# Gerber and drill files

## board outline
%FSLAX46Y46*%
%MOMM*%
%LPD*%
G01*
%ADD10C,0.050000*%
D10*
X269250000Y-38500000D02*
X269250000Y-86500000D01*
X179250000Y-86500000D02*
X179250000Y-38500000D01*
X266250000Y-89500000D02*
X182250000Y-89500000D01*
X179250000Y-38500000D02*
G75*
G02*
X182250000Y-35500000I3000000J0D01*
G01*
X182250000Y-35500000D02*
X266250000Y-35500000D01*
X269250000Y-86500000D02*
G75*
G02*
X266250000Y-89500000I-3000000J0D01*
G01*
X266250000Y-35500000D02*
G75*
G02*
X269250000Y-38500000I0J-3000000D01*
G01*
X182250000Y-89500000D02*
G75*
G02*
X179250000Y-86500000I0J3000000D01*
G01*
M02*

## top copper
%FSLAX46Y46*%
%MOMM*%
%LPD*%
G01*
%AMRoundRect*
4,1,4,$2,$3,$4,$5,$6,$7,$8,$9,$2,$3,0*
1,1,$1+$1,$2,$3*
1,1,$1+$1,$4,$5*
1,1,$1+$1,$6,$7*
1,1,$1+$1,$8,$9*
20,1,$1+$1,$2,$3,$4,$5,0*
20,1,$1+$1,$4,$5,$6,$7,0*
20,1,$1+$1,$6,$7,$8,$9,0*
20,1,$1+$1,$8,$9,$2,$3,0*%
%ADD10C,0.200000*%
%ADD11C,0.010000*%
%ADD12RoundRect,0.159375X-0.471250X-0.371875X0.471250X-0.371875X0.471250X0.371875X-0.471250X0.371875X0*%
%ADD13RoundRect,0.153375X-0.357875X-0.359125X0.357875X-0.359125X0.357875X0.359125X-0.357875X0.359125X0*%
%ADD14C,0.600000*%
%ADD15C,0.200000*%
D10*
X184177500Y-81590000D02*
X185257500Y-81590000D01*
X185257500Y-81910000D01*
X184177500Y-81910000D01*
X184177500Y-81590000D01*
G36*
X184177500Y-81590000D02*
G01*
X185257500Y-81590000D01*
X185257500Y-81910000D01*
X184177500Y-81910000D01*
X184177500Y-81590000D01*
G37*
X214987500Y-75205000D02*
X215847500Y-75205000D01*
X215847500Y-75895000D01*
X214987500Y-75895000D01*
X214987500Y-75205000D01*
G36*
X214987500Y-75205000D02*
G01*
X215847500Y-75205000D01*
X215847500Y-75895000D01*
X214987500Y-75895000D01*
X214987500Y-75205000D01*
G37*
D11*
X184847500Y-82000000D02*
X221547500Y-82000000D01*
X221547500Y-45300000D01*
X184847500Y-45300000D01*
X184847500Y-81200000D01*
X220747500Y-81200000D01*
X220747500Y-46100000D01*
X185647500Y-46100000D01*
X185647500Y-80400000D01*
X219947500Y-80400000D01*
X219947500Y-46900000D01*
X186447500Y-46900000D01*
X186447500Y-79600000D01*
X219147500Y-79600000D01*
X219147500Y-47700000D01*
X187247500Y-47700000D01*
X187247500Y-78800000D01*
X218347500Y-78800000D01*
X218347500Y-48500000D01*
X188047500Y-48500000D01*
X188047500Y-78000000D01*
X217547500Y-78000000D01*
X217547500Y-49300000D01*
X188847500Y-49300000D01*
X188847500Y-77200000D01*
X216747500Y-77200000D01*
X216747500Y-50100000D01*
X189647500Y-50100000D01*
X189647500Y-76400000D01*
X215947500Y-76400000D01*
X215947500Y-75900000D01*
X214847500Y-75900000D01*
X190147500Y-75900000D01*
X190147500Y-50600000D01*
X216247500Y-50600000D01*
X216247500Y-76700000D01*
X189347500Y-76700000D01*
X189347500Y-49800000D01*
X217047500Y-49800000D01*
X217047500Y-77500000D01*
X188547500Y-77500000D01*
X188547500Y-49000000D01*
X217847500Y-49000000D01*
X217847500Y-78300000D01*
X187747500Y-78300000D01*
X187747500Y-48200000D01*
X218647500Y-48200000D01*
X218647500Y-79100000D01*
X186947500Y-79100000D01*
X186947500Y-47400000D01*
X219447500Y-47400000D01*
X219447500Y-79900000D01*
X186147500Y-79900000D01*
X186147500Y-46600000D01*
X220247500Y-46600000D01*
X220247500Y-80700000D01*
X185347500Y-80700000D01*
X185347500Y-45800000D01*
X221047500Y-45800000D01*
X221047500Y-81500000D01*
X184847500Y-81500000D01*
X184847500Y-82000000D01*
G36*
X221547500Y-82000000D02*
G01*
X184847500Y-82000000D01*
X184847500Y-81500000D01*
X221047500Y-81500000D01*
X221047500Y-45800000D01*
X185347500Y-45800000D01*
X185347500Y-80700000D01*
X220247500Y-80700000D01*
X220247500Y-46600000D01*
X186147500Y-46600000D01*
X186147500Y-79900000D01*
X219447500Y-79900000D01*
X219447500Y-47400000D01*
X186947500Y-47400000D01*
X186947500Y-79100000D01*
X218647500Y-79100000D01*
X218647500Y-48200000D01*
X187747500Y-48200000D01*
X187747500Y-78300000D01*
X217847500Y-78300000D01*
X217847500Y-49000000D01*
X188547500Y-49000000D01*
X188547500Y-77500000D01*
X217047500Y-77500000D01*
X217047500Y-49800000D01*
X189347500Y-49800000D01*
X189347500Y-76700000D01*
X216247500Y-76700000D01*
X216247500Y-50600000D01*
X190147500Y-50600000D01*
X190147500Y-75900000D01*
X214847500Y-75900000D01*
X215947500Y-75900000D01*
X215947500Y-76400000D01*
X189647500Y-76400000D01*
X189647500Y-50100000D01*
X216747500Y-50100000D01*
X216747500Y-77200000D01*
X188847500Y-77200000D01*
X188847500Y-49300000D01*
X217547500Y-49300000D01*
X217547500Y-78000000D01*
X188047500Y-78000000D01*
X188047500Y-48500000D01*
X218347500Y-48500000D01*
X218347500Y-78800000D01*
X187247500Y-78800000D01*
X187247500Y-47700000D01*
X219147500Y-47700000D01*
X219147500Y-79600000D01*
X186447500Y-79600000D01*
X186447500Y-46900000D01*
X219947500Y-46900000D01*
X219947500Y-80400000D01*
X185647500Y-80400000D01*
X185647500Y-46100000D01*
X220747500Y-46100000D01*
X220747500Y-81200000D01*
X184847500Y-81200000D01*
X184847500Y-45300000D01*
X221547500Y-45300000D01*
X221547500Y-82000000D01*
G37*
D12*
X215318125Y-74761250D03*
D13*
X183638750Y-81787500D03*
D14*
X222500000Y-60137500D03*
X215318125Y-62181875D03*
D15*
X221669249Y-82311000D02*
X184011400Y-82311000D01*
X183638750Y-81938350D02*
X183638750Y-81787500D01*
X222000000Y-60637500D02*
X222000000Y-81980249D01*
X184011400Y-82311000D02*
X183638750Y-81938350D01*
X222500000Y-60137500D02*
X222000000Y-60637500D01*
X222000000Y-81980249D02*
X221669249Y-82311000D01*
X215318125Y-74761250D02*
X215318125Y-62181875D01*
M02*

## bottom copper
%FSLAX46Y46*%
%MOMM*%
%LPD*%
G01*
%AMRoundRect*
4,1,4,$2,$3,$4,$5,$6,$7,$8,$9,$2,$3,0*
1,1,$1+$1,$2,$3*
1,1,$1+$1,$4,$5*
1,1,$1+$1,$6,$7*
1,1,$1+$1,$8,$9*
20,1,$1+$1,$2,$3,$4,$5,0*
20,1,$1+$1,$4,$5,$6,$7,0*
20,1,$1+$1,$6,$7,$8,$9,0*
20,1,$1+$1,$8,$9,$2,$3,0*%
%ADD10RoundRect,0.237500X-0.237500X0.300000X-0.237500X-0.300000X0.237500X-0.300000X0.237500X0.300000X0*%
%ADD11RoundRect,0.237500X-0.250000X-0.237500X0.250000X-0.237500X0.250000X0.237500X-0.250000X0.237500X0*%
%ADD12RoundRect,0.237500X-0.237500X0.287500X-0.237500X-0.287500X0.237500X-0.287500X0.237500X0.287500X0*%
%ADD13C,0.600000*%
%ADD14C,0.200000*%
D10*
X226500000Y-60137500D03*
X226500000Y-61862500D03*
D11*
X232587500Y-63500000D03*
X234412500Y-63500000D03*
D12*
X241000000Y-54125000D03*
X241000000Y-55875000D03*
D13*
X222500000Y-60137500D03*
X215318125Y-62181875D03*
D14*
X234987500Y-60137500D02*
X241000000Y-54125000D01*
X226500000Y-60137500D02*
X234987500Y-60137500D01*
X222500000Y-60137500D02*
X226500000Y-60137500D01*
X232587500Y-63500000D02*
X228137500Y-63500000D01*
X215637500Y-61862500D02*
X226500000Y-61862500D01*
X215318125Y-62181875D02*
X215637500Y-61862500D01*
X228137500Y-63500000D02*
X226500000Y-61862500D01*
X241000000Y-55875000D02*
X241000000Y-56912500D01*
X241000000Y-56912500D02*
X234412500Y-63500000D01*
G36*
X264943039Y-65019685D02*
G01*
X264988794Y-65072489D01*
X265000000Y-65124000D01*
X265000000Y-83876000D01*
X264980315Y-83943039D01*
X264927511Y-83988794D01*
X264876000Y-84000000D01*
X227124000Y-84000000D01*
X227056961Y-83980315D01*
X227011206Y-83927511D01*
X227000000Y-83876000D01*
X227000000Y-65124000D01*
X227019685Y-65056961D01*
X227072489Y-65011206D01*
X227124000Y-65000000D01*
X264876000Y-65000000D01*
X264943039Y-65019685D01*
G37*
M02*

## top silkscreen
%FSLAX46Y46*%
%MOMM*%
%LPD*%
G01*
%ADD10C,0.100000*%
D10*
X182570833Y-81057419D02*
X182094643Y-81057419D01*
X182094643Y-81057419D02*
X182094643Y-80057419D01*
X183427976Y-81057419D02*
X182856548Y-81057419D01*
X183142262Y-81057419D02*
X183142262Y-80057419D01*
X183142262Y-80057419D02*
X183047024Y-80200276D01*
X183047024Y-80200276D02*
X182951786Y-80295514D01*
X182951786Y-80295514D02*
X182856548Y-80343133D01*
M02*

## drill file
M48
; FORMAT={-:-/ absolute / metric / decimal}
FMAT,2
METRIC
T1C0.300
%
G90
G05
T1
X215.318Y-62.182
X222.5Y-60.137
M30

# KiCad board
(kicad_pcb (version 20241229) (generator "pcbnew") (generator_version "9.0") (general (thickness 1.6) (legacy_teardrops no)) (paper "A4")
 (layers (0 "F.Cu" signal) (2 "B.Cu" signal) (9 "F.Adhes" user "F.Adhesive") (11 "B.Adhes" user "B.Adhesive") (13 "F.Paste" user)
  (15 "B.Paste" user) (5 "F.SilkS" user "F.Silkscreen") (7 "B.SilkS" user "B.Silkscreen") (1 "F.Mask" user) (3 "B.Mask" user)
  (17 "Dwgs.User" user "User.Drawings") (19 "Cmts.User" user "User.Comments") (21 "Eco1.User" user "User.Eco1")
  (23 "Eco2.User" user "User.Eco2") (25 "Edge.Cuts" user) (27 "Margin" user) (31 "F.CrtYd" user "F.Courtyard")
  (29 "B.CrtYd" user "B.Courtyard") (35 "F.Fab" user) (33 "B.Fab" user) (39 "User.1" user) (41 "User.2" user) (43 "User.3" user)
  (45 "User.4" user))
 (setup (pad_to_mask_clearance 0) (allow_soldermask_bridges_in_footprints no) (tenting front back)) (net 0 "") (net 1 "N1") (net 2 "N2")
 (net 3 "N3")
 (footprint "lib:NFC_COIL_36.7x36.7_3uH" (layer "F.Cu") (at 184.8475 82)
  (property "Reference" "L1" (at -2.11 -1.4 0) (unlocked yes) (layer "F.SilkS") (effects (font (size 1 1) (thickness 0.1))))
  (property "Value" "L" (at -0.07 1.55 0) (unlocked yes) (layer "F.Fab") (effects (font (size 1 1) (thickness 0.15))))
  (fp_rect (start -0.67 -0.41) (end 0.41 -0.09) (stroke (width 0.2) (type solid)) (fill yes) (layer "F.Cu"))
  (fp_rect (start 30.14 -6.795) (end 31 -6.105) (stroke (width 0.2) (type solid)) (fill yes) (layer "F.Cu"))
  (fp_poly
   (pts (xy 0 0) (xy 36.7 0) (xy 36.7 -36.7) (xy 0 -36.7) (xy 0 -0.8) (xy 35.9 -0.8) (xy 35.9 -35.9) (xy 0.8 -35.9) (xy 0.8 -1.6)
    (xy 35.1 -1.6) (xy 35.1 -35.1) (xy 1.6 -35.1) (xy 1.6 -2.4) (xy 34.3 -2.4) (xy 34.3 -34.3) (xy 2.4 -34.3) (xy 2.4 -3.2) (xy 33.5 -3.2)
    (xy 33.5 -33.5) (xy 3.2 -33.5) (xy 3.2 -4) (xy 32.7 -4) (xy 32.7 -32.7) (xy 4 -32.7) (xy 4 -4.8) (xy 31.9 -4.8) (xy 31.9 -31.9)
    (xy 4.8 -31.9) (xy 4.8 -5.6) (xy 31.1 -5.6) (xy 31.1 -6.1) (xy 30 -6.1) (xy 5.3 -6.1) (xy 5.3 -31.4) (xy 31.4 -31.4) (xy 31.4 -5.3)
    (xy 4.5 -5.3) (xy 4.5 -32.2) (xy 32.2 -32.2) (xy 32.2 -4.5) (xy 3.7 -4.5) (xy 3.7 -33) (xy 33 -33) (xy 33 -3.7) (xy 2.9 -3.7)
    (xy 2.9 -33.8) (xy 33.8 -33.8) (xy 33.8 -2.9) (xy 2.1 -2.9) (xy 2.1 -34.6) (xy 34.6 -34.6) (xy 34.6 -2.1) (xy 1.3 -2.1) (xy 1.3 -35.4)
    (xy 35.4 -35.4) (xy 35.4 -1.3) (xy 0.5 -1.3) (xy 0.5 -36.2) (xy 36.2 -36.2) (xy 36.2 -0.5) (xy 0 -0.5))
   (stroke (width 0.01) (type solid)) (fill yes) (layer "F.Cu"))
  (pad "1" smd roundrect (at 30.470625 -7.23875) (size 1.26125 1.0625) (layers "F.Cu" "F.Mask" "F.Paste") (roundrect_rratio 0.15)
   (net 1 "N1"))
  (pad "2" smd roundrect (at -1.20875 -0.2125) (size 1.0225 1.025) (layers "F.Cu" "F.Mask" "F.Paste") (roundrect_rratio 0.15) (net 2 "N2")))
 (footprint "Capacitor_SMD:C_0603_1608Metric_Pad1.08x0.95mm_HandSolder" (layer "B.Cu") (at 226.5 61 -90)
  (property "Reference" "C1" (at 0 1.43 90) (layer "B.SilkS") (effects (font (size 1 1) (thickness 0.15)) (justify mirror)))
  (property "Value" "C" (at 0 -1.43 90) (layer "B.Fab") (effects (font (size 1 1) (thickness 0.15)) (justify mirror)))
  (pad "1" smd roundrect (at -0.8625 0 270) (size 1.075 0.95) (layers "B.Cu" "B.Mask" "B.Paste") (roundrect_rratio 0.25) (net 2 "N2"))
  (pad "2" smd roundrect (at 0.8625 0 270) (size 1.075 0.95) (layers "B.Cu" "B.Mask" "B.Paste") (roundrect_rratio 0.25) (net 1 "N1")))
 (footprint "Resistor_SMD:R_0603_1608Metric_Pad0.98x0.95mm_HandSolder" (layer "B.Cu") (at 233.5 63.5)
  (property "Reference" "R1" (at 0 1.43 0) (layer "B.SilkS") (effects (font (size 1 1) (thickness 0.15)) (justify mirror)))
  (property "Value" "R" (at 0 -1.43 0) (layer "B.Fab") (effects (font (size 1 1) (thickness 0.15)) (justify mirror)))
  (pad "1" smd roundrect (at -0.9125 0) (size 0.975 0.95) (layers "B.Cu" "B.Mask" "B.Paste") (roundrect_rratio 0.25) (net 1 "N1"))
  (pad "2" smd roundrect (at 0.9125 0) (size 0.975 0.95) (layers "B.Cu" "B.Mask" "B.Paste") (roundrect_rratio 0.25) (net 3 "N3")))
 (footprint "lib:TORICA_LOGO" (layer "B.Cu") (at 246 48.5 180)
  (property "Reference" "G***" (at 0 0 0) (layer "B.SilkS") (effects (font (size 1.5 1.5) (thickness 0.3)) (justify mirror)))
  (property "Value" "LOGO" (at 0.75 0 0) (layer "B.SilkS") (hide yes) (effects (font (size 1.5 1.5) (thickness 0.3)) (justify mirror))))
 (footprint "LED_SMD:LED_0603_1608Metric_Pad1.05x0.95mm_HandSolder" (layer "B.Cu") (at 241 55 -90)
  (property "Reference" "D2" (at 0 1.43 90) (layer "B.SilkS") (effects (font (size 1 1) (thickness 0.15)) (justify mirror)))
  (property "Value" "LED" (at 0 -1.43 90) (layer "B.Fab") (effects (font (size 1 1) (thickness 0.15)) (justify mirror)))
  (pad "1" smd roundrect (at -0.875 0 270) (size 1.05 0.95) (layers "B.Cu" "B.Mask" "B.Paste") (roundrect_rratio 0.25) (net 2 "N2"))
  (pad "2" smd roundrect (at 0.875 0 270) (size 1.05 0.95) (layers "B.Cu" "B.Mask" "B.Paste") (roundrect_rratio 0.25) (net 3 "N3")))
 (gr_line (start 269.25 38.5) (end 269.25 86.5) (stroke (width 0.05) (type default)) (layer "Edge.Cuts"))
 (gr_line (start 179.25 86.5) (end 179.25 38.5) (stroke (width 0.05) (type default)) (layer "Edge.Cuts"))
 (gr_line (start 266.25 89.5) (end 182.25 89.5) (stroke (width 0.05) (type default)) (layer "Edge.Cuts"))
 (gr_arc (start 179.25 38.5) (mid 180.12868 36.37868) (end 182.25 35.5) (stroke (width 0.05) (type default)) (layer "Edge.Cuts"))
 (gr_line (start 182.25 35.5) (end 266.25 35.5) (stroke (width 0.05) (type default)) (layer "Edge.Cuts"))
 (gr_arc (start 269.25 86.5) (mid 268.37132 88.62132) (end 266.25 89.5) (stroke (width 0.05) (type default)) (layer "Edge.Cuts"))
 (gr_arc (start 266.25 35.5) (mid 268.37132 36.37868) (end 269.25 38.5) (stroke (width 0.05) (type default)) (layer "Edge.Cuts"))
 (gr_arc (start 182.25 89.5) (mid 180.12868 88.62132) (end 179.25 86.5) (stroke (width 0.05) (type default)) (layer "Edge.Cuts"))
 (segment (start 221.669249 82.311) (end 184.0114 82.311) (width 0.2) (layer "F.Cu") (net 2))
 (segment (start 183.63875 81.93835) (end 183.63875 81.7875) (width 0.2) (layer "F.Cu") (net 2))
 (segment (start 222 60.6375) (end 222 81.980249) (width 0.2) (layer "F.Cu") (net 2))
 (segment (start 184.0114 82.311) (end 183.63875 81.93835) (width 0.2) (layer "F.Cu") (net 2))
 (segment (start 222.5 60.1375) (end 222 60.6375) (width 0.2) (layer "F.Cu") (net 2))
 (segment (start 222 81.980249) (end 221.669249 82.311) (width 0.2) (layer "F.Cu") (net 2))
 (via (at 222.5 60.1375) (size 0.6) (drill 0.3) (layers "F.Cu" "B.Cu") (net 2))
 (segment (start 234.9875 60.1375) (end 241 54.125) (width 0.2) (layer "B.Cu") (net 2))
 (segment (start 226.5 60.1375) (end 234.9875 60.1375) (width 0.2) (layer "B.Cu") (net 2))
 (segment (start 222.5 60.1375) (end 226.5 60.1375) (width 0.2) (layer "B.Cu") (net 2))
 (segment (start 215.318125 74.76125) (end 215.318125 62.181875) (width 0.2) (layer "F.Cu") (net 1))
 (via (at 215.318125 62.181875) (size 0.6) (drill 0.3) (layers "F.Cu" "B.Cu") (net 1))
 (segment (start 232.5875 63.5) (end 228.1375 63.5) (width 0.2) (layer "B.Cu") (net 1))
 (segment (start 215.6375 61.8625) (end 226.5 61.8625) (width 0.2) (layer "B.Cu") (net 1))
 (segment (start 215.318125 62.181875) (end 215.6375 61.8625) (width 0.2) (layer "B.Cu") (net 1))
 (segment (start 228.1375 63.5) (end 226.5 61.8625) (width 0.2) (layer "B.Cu") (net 1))
 (segment (start 241 55.875) (end 241 56.9125) (width 0.2) (layer "B.Cu") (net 3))
 (segment (start 241 56.9125) (end 234.4125 63.5) (width 0.2) (layer "B.Cu") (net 3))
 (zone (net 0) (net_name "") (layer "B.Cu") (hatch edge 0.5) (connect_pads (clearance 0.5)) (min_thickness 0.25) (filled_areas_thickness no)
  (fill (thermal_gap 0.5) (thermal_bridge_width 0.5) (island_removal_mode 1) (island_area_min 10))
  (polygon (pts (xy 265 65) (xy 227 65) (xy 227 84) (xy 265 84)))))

